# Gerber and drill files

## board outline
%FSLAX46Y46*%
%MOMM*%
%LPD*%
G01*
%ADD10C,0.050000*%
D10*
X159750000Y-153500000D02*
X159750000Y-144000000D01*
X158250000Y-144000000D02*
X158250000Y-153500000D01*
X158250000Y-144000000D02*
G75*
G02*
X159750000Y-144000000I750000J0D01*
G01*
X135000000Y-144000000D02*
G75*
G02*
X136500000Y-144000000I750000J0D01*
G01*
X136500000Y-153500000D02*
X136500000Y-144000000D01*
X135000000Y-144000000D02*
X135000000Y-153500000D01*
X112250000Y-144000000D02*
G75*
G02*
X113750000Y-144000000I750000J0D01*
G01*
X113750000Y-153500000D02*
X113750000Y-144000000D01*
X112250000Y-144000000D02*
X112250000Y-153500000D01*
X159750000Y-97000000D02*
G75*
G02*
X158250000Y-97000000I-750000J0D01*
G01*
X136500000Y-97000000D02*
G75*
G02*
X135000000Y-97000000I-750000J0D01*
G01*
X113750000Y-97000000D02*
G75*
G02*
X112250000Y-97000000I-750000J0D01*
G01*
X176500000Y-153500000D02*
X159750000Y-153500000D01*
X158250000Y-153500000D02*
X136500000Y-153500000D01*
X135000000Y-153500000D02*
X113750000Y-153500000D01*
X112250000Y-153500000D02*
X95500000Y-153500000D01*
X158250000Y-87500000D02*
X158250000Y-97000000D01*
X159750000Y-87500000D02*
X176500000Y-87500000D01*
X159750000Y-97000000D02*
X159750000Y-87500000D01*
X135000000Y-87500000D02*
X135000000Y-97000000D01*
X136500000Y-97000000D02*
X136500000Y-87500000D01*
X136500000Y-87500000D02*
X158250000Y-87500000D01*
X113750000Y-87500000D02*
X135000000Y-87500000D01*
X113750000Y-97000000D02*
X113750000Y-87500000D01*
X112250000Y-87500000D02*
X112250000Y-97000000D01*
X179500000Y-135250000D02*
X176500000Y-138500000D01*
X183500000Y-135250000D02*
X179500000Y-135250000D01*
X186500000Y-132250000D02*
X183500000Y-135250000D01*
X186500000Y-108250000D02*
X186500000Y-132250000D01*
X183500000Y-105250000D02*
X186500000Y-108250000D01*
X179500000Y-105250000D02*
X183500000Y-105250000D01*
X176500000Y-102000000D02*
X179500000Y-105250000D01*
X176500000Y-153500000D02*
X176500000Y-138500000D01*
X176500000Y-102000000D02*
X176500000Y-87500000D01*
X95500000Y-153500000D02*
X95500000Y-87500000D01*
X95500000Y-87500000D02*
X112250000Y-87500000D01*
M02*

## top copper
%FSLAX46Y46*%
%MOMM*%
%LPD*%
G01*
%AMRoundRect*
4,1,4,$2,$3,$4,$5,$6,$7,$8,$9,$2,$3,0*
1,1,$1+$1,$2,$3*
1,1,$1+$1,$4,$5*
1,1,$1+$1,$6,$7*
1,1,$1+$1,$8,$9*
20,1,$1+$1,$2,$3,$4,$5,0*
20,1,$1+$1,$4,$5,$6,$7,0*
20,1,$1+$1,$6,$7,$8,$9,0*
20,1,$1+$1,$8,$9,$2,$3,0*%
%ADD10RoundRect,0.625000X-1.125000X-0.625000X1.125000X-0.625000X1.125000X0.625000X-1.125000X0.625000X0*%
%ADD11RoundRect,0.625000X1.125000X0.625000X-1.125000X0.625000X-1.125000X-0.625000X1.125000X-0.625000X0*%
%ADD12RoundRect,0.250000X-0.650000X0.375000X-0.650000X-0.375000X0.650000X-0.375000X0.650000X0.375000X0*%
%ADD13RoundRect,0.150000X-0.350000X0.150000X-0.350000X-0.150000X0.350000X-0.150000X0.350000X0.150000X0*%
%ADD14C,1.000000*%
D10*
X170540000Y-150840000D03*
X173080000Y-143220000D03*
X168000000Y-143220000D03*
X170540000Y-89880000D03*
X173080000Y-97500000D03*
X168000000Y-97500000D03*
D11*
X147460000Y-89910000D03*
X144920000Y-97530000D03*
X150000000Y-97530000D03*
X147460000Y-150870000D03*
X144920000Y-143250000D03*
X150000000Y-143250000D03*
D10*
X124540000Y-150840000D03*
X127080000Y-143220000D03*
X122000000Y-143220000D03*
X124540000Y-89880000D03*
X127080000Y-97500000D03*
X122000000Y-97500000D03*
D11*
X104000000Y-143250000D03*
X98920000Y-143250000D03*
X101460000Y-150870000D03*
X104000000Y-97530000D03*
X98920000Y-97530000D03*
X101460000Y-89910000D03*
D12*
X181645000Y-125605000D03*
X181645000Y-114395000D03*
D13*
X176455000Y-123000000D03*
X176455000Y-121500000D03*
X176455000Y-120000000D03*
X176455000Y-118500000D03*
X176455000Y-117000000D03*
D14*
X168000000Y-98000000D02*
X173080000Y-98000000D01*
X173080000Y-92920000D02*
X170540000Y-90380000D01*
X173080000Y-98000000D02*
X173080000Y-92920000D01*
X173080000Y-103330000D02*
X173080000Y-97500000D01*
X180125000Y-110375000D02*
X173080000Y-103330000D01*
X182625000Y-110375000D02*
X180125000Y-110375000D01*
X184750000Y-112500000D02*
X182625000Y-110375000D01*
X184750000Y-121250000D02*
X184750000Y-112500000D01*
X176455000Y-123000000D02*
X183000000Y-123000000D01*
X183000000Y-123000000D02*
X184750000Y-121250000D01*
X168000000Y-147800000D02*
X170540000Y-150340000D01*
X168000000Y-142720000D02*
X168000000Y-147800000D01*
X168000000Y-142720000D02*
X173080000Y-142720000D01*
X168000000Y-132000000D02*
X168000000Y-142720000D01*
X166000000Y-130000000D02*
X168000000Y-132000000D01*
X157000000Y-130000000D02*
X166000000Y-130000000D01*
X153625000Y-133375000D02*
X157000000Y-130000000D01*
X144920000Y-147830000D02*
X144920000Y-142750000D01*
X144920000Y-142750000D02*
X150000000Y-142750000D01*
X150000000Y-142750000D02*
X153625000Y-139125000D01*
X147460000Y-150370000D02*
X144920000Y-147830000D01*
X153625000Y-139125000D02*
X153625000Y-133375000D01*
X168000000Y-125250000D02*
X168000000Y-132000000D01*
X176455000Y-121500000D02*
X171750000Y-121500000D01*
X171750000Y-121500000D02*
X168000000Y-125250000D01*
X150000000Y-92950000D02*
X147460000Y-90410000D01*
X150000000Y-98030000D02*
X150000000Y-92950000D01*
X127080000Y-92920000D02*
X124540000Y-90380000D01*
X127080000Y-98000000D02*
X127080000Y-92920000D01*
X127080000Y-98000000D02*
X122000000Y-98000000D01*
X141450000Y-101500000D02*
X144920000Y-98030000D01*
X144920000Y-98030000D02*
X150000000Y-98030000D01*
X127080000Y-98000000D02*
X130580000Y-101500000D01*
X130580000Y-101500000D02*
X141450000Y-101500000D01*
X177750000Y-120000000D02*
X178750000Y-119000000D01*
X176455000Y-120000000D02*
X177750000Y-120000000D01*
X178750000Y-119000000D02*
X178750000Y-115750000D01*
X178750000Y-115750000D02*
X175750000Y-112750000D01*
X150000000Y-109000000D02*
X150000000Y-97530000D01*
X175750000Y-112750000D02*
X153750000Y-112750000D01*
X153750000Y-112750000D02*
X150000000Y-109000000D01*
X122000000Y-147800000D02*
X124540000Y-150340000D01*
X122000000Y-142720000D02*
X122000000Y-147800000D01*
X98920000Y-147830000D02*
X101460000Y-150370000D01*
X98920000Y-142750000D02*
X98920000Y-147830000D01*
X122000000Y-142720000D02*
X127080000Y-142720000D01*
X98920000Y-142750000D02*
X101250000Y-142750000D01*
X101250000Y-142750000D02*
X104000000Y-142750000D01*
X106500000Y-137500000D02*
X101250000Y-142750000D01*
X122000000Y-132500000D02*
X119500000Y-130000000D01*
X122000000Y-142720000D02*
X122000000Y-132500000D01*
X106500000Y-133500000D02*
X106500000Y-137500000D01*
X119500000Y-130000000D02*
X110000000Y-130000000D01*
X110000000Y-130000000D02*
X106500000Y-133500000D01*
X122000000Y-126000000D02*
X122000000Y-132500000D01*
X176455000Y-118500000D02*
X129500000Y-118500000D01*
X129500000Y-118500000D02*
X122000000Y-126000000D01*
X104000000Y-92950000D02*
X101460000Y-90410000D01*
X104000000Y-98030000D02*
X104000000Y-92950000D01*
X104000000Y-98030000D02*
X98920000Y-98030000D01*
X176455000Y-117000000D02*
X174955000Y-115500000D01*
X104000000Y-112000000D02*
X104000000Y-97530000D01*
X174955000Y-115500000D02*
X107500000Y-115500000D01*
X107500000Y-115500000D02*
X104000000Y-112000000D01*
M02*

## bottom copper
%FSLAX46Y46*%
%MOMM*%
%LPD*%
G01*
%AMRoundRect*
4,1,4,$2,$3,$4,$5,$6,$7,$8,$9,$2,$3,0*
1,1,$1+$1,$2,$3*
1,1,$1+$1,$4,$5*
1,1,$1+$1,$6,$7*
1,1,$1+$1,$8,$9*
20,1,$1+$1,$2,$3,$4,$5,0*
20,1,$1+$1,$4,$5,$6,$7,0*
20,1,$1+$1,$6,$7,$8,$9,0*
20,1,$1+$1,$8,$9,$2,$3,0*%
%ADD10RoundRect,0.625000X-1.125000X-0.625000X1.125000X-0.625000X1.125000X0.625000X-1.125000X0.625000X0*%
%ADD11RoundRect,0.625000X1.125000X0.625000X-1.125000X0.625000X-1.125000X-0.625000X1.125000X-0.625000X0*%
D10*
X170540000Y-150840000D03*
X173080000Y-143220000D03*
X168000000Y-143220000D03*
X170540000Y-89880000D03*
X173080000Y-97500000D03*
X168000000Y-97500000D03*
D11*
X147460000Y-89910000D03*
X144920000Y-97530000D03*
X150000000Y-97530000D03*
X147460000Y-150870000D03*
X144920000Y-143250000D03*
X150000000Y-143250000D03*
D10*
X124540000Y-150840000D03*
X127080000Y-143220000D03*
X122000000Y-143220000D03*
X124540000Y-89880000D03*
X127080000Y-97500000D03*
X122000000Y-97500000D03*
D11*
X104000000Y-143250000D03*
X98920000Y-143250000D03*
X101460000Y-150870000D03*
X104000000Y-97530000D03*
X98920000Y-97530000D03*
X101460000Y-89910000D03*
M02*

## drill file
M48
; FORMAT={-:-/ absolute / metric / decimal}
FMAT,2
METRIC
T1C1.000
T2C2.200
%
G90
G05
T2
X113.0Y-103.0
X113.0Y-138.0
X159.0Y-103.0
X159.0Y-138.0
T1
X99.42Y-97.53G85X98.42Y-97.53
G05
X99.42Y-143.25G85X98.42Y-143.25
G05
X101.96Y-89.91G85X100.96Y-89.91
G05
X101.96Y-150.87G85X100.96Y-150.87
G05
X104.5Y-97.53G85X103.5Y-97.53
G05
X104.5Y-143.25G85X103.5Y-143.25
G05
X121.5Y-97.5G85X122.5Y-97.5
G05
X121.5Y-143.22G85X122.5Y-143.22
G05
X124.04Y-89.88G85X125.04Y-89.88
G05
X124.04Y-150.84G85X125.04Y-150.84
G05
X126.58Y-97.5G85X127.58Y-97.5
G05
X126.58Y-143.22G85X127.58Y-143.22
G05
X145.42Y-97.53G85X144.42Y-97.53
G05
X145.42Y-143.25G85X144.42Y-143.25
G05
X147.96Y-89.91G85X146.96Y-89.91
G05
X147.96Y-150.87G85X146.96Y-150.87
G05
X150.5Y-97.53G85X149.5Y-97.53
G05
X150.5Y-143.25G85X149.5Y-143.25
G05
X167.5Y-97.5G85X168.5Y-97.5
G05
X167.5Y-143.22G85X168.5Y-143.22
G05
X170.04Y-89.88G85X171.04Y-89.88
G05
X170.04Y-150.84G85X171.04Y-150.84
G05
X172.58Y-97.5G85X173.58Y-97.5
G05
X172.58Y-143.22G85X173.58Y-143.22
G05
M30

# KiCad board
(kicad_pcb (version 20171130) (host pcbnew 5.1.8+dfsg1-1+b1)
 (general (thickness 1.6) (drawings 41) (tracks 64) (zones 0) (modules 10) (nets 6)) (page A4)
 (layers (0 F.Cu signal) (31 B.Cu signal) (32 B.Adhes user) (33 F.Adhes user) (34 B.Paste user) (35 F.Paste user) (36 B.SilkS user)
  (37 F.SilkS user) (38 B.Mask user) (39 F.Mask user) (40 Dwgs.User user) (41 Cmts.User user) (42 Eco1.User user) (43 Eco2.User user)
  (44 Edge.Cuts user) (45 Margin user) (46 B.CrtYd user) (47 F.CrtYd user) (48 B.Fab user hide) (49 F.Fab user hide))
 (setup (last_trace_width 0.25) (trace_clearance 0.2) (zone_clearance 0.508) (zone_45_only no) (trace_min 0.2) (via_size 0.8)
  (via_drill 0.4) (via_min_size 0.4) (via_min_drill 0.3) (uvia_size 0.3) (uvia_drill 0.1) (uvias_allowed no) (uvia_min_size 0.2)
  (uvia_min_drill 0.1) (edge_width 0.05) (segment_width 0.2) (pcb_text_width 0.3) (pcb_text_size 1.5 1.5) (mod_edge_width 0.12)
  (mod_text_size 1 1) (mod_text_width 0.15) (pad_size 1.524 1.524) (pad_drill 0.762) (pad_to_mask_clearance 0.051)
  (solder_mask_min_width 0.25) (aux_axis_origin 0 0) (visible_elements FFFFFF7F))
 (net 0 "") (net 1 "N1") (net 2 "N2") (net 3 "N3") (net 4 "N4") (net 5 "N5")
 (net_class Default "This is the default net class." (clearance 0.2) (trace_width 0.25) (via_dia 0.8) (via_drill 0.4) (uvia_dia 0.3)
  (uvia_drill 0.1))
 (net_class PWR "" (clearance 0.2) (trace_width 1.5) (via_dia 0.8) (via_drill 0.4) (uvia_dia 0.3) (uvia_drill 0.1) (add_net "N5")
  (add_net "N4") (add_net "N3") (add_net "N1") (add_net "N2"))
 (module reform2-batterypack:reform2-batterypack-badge (layer F.Cu) (at 136 120.5 90)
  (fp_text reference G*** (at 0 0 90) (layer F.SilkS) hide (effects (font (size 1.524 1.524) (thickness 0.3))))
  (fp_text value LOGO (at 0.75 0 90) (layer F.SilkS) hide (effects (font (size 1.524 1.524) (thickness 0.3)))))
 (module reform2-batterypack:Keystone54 (layer F.Cu) (at 168 98)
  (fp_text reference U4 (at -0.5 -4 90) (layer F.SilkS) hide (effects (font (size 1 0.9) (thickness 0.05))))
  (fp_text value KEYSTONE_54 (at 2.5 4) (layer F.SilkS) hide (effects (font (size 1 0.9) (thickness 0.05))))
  (pad 6 thru_hole roundrect (at 2.54 52.84) (size 3.5 2.5) (drill oval 2 1) (layers *.Cu *.Mask) (roundrect_rratio 0.25) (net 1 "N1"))
  (pad 5 thru_hole roundrect (at 5.08 45.22) (size 3.5 2.5) (drill oval 2 1) (layers *.Cu *.Mask) (roundrect_rratio 0.25) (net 1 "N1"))
  (pad 4 thru_hole roundrect (at 0 45.22) (size 3.5 2.5) (drill oval 2 1) (layers *.Cu *.Mask) (roundrect_rratio 0.25) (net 1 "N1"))
  (pad 3 thru_hole roundrect (at 2.54 -8.12) (size 3.5 2.5) (drill oval 2 1) (layers *.Cu *.Mask) (roundrect_rratio 0.25) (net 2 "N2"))
  (pad 2 thru_hole roundrect (at 5.08 -0.5) (size 3.5 2.5) (drill oval 2 1) (layers *.Cu *.Mask) (roundrect_rratio 0.25) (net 2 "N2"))
  (pad 1 thru_hole roundrect (at 0 -0.5) (size 3.5 2.5) (drill oval 2 1) (layers *.Cu *.Mask) (roundrect_rratio 0.25) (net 2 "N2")))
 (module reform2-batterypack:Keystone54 (layer F.Cu) (at 150 142.75 180)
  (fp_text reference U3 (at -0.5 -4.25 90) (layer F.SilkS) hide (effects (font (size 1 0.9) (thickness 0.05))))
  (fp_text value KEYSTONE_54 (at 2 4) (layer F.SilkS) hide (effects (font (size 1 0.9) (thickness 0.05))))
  (pad 6 thru_hole roundrect (at 2.54 52.84 180) (size 3.5 2.5) (drill oval 2 1) (layers *.Cu *.Mask) (roundrect_rratio 0.25) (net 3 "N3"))
  (pad 5 thru_hole roundrect (at 5.08 45.22 180) (size 3.5 2.5) (drill oval 2 1) (layers *.Cu *.Mask) (roundrect_rratio 0.25) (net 3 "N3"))
  (pad 4 thru_hole roundrect (at 0 45.22 180) (size 3.5 2.5) (drill oval 2 1) (layers *.Cu *.Mask) (roundrect_rratio 0.25) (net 3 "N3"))
  (pad 3 thru_hole roundrect (at 2.54 -8.12 180) (size 3.5 2.5) (drill oval 2 1) (layers *.Cu *.Mask) (roundrect_rratio 0.25) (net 1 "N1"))
  (pad 2 thru_hole roundrect (at 5.08 -0.5 180) (size 3.5 2.5) (drill oval 2 1) (layers *.Cu *.Mask) (roundrect_rratio 0.25) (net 1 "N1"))
  (pad 1 thru_hole roundrect (at 0 -0.5 180) (size 3.5 2.5) (drill oval 2 1) (layers *.Cu *.Mask) (roundrect_rratio 0.25) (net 1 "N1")))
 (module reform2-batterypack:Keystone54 (layer F.Cu) (at 122 98)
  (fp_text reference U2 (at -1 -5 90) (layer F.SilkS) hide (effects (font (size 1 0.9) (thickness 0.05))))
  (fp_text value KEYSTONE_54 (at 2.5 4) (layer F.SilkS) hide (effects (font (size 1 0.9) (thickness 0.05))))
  (pad 6 thru_hole roundrect (at 2.54 52.84) (size 3.5 2.5) (drill oval 2 1) (layers *.Cu *.Mask) (roundrect_rratio 0.25) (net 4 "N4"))
  (pad 5 thru_hole roundrect (at 5.08 45.22) (size 3.5 2.5) (drill oval 2 1) (layers *.Cu *.Mask) (roundrect_rratio 0.25) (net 4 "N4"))
  (pad 4 thru_hole roundrect (at 0 45.22) (size 3.5 2.5) (drill oval 2 1) (layers *.Cu *.Mask) (roundrect_rratio 0.25) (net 4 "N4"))
  (pad 3 thru_hole roundrect (at 2.54 -8.12) (size 3.5 2.5) (drill oval 2 1) (layers *.Cu *.Mask) (roundrect_rratio 0.25) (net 3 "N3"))
  (pad 2 thru_hole roundrect (at 5.08 -0.5) (size 3.5 2.5) (drill oval 2 1) (layers *.Cu *.Mask) (roundrect_rratio 0.25) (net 3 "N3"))
  (pad 1 thru_hole roundrect (at 0 -0.5) (size 3.5 2.5) (drill oval 2 1) (layers *.Cu *.Mask) (roundrect_rratio 0.25) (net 3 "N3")))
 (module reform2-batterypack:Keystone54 (layer F.Cu) (at 104 142.75 180)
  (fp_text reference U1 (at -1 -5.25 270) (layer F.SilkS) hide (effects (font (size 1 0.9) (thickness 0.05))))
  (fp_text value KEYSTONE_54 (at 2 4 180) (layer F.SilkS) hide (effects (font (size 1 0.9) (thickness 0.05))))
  (pad 1 thru_hole roundrect (at 0 -0.5 180) (size 3.5 2.5) (drill oval 2 1) (layers *.Cu *.Mask) (roundrect_rratio 0.25) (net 4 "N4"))
  (pad 2 thru_hole roundrect (at 5.08 -0.5 180) (size 3.5 2.5) (drill oval 2 1) (layers *.Cu *.Mask) (roundrect_rratio 0.25) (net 4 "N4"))
  (pad 3 thru_hole roundrect (at 2.54 -8.12 180) (size 3.5 2.5) (drill oval 2 1) (layers *.Cu *.Mask) (roundrect_rratio 0.25) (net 4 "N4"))
  (pad 4 thru_hole roundrect (at 0 45.22 180) (size 3.5 2.5) (drill oval 2 1) (layers *.Cu *.Mask) (roundrect_rratio 0.25) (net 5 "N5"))
  (pad 5 thru_hole roundrect (at 5.08 45.22 180) (size 3.5 2.5) (drill oval 2 1) (layers *.Cu *.Mask) (roundrect_rratio 0.25) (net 5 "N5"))
  (pad 6 thru_hole roundrect (at 2.54 52.84 180) (size 3.5 2.5) (drill oval 2 1) (layers *.Cu *.Mask) (roundrect_rratio 0.25) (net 5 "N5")))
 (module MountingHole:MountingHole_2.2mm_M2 (layer F.Cu) (at 159 138)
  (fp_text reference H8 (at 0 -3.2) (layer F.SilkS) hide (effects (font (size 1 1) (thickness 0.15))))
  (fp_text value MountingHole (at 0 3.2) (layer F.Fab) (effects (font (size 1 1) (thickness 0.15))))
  (pad 1 np_thru_hole circle (at 0 0) (size 2.2 2.2) (drill 2.2) (layers *.Cu *.Mask)))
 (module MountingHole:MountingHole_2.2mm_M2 (layer F.Cu) (at 113 138)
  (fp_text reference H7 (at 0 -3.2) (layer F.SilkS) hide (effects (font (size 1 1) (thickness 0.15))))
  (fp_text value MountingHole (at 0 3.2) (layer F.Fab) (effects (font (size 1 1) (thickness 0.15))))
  (pad 1 np_thru_hole circle (at 0 0) (size 2.2 2.2) (drill 2.2) (layers *.Cu *.Mask)))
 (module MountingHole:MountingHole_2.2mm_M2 (layer F.Cu) (at 159 103)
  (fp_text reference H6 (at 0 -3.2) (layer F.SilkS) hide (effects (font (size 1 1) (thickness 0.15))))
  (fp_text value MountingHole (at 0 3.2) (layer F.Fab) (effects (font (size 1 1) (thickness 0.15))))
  (pad 1 np_thru_hole circle (at 0 0) (size 2.2 2.2) (drill 2.2) (layers *.Cu *.Mask)))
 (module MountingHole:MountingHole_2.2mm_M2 (layer F.Cu) (at 113 103)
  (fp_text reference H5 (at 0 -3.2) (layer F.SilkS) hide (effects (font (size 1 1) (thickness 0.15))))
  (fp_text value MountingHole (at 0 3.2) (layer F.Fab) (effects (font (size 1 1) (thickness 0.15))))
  (pad 1 np_thru_hole circle (at 0 0) (size 2.2 2.2) (drill 2.2) (layers *.Cu *.Mask)))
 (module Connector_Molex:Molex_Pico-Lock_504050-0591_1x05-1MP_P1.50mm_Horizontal (layer F.Cu) (at 179.25 120 270)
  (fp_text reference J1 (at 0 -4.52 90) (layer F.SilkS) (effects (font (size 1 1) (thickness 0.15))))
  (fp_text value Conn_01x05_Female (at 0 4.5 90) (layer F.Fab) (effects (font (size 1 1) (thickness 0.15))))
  (pad MP smd roundrect (at 5.605 -2.395 270) (size 1.25 1.8) (layers F.Cu F.Paste F.Mask) (roundrect_rratio 0.2))
  (pad MP smd roundrect (at -5.605 -2.395 270) (size 1.25 1.8) (layers F.Cu F.Paste F.Mask) (roundrect_rratio 0.2))
  (pad 5 smd roundrect (at 3 2.795 270) (size 0.6 1) (layers F.Cu F.Paste F.Mask) (roundrect_rratio 0.25) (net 2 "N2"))
  (pad 4 smd roundrect (at 1.5 2.795 270) (size 0.6 1) (layers F.Cu F.Paste F.Mask) (roundrect_rratio 0.25) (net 1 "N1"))
  (pad 3 smd roundrect (at 0 2.795 270) (size 0.6 1) (layers F.Cu F.Paste F.Mask) (roundrect_rratio 0.25) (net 3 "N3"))
  (pad 2 smd roundrect (at -1.5 2.795 270) (size 0.6 1) (layers F.Cu F.Paste F.Mask) (roundrect_rratio 0.25) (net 4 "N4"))
  (pad 1 smd roundrect (at -3 2.795 270) (size 0.6 1) (layers F.Cu F.Paste F.Mask) (roundrect_rratio 0.25) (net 5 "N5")))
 (gr_line (start 159.75 153.5) (end 159.75 144) (layer Edge.Cuts) (width 0.05))
 (gr_line (start 158.25 144) (end 158.25 153.5) (layer Edge.Cuts) (width 0.05))
 (gr_arc (start 159 144) (end 159.75 144) (angle -180) (layer Edge.Cuts) (width 0.05))
 (gr_arc (start 135.75 144) (end 136.5 144) (angle -180) (layer Edge.Cuts) (width 0.05))
 (gr_line (start 136.5 153.5) (end 136.5 144) (layer Edge.Cuts) (width 0.05))
 (gr_line (start 135 144) (end 135 153.5) (layer Edge.Cuts) (width 0.05))
 (gr_arc (start 113 144) (end 113.75 144) (angle -180) (layer Edge.Cuts) (width 0.05))
 (gr_line (start 113.75 153.5) (end 113.75 144) (layer Edge.Cuts) (width 0.05))
 (gr_line (start 112.25 144) (end 112.25 153.5) (layer Edge.Cuts) (width 0.05))
 (gr_arc (start 159 97) (end 158.25 97) (angle -180) (layer Edge.Cuts) (width 0.05))
 (gr_arc (start 135.75 97) (end 135 97) (angle -180) (layer Edge.Cuts) (width 0.05))
 (gr_arc (start 113 97) (end 112.25 97) (angle -180) (layer Edge.Cuts) (width 0.05))
 (gr_line (start 176.5 153.5) (end 159.75 153.5) (layer Edge.Cuts) (width 0.05))
 (gr_line (start 158.25 153.5) (end 136.5 153.5) (layer Edge.Cuts) (width 0.05))
 (gr_line (start 135 153.5) (end 113.75 153.5) (layer Edge.Cuts) (width 0.05))
 (gr_line (start 112.25 153.5) (end 95.5 153.5) (layer Edge.Cuts) (width 0.05))
 (gr_line (start 158.25 87.5) (end 158.25 97) (layer Edge.Cuts) (width 0.05))
 (gr_line (start 159.75 87.5) (end 176.5 87.5) (layer Edge.Cuts) (width 0.05))
 (gr_line (start 159.75 97) (end 159.75 87.5) (layer Edge.Cuts) (width 0.05))
 (gr_line (start 135 87.5) (end 135 97) (layer Edge.Cuts) (width 0.05))
 (gr_line (start 136.5 97) (end 136.5 87.5) (layer Edge.Cuts) (width 0.05))
 (gr_line (start 136.5 87.5) (end 158.25 87.5) (layer Edge.Cuts) (width 0.05))
 (gr_line (start 113.75 87.5) (end 135 87.5) (layer Edge.Cuts) (width 0.05))
 (gr_line (start 113.75 97) (end 113.75 87.5) (layer Edge.Cuts) (width 0.05))
 (gr_line (start 112.25 87.5) (end 112.25 97) (layer Edge.Cuts) (width 0.05))
 (gr_line (start 179.5 135.25) (end 176.5 138.5) (layer Edge.Cuts) (width 0.05))
 (gr_line (start 183.5 135.25) (end 179.5 135.25) (layer Edge.Cuts) (width 0.05))
 (gr_line (start 186.5 132.25) (end 183.5 135.25) (layer Edge.Cuts) (width 0.05))
 (gr_line (start 186.5 108.25) (end 186.5 132.25) (layer Edge.Cuts) (width 0.05))
 (gr_line (start 183.5 105.25) (end 186.5 108.25) (layer Edge.Cuts) (width 0.05))
 (gr_line (start 179.5 105.25) (end 183.5 105.25) (layer Edge.Cuts) (width 0.05))
 (gr_line (start 176.5 102) (end 179.5 105.25) (layer Edge.Cuts) (width 0.05))
 (gr_line (start 176.5 153.5) (end 176.5 138.5) (layer Edge.Cuts) (width 0.05))
 (gr_line (start 176.5 102) (end 176.5 87.5) (layer Edge.Cuts) (width 0.05))
 (gr_line (start 95.5 153.5) (end 95.5 87.5) (layer Edge.Cuts) (width 0.05))
 (gr_line (start 95.5 87.5) (end 112.25 87.5) (layer Edge.Cuts) (width 0.05))
 (segment (start 168 98) (end 173.08 98) (width 1) (layer F.Cu) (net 2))
 (segment (start 173.08 92.92) (end 170.54 90.38) (width 1) (layer F.Cu) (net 2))
 (segment (start 173.08 98) (end 173.08 92.92) (width 1) (layer F.Cu) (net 2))
 (segment (start 173.08 103.33) (end 173.08 97.5) (width 1) (layer F.Cu) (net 2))
 (segment (start 180.125 110.375) (end 173.08 103.33) (width 1) (layer F.Cu) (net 2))
 (segment (start 182.625 110.375) (end 180.125 110.375) (width 1) (layer F.Cu) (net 2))
 (segment (start 184.75 112.5) (end 182.625 110.375) (width 1) (layer F.Cu) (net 2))
 (segment (start 184.75 121.25) (end 184.75 112.5) (width 1) (layer F.Cu) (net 2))
 (segment (start 176.455 123) (end 183 123) (width 1) (layer F.Cu) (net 2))
 (segment (start 183 123) (end 184.75 121.25) (width 1) (layer F.Cu) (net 2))
 (segment (start 168 147.8) (end 170.54 150.34) (width 1) (layer F.Cu) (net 1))
 (segment (start 168 142.72) (end 168 147.8) (width 1) (layer F.Cu) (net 1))
 (segment (start 168 142.72) (end 173.08 142.72) (width 1) (layer F.Cu) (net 1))
 (segment (start 168 132) (end 168 142.72) (width 1) (layer F.Cu) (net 1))
 (segment (start 166 130) (end 168 132) (width 1) (layer F.Cu) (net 1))
 (segment (start 157 130) (end 166 130) (width 1) (layer F.Cu) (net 1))
 (segment (start 153.625 133.375) (end 157 130) (width 1) (layer F.Cu) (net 1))
 (segment (start 144.92 147.83) (end 144.92 142.75) (width 1) (layer F.Cu) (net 1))
 (segment (start 144.92 142.75) (end 150 142.75) (width 1) (layer F.Cu) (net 1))
 (segment (start 150 142.75) (end 153.625 139.125) (width 1) (layer F.Cu) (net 1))
 (segment (start 147.46 150.37) (end 144.92 147.83) (width 1) (layer F.Cu) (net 1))
 (segment (start 153.625 139.125) (end 153.625 133.375) (width 1) (layer F.Cu) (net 1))
 (segment (start 168 125.25) (end 168 132) (width 1) (layer F.Cu) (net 1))
 (segment (start 176.455 121.5) (end 171.75 121.5) (width 1) (layer F.Cu) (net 1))
 (segment (start 171.75 121.5) (end 168 125.25) (width 1) (layer F.Cu) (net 1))
 (segment (start 150 92.95) (end 147.46 90.41) (width 1) (layer F.Cu) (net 3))
 (segment (start 150 98.03) (end 150 92.95) (width 1) (layer F.Cu) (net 3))
 (segment (start 127.08 92.92) (end 124.54 90.38) (width 1) (layer F.Cu) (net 3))
 (segment (start 127.08 98) (end 127.08 92.92) (width 1) (layer F.Cu) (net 3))
 (segment (start 127.08 98) (end 122 98) (width 1) (layer F.Cu) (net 3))
 (segment (start 141.45 101.5) (end 144.92 98.03) (width 1) (layer F.Cu) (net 3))
 (segment (start 144.92 98.03) (end 150 98.03) (width 1) (layer F.Cu) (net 3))
 (segment (start 127.08 98) (end 130.58 101.5) (width 1) (layer F.Cu) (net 3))
 (segment (start 130.58 101.5) (end 141.45 101.5) (width 1) (layer F.Cu) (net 3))
 (segment (start 177.75 120) (end 178.75 119) (width 1) (layer F.Cu) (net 3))
 (segment (start 176.455 120) (end 177.75 120) (width 1) (layer F.Cu) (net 3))
 (segment (start 178.75 119) (end 178.75 115.75) (width 1) (layer F.Cu) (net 3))
 (segment (start 178.75 115.75) (end 175.75 112.75) (width 1) (layer F.Cu) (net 3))
 (segment (start 150 109) (end 150 97.53) (width 1) (layer F.Cu) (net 3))
 (segment (start 175.75 112.75) (end 153.75 112.75) (width 1) (layer F.Cu) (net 3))
 (segment (start 153.75 112.75) (end 150 109) (width 1) (layer F.Cu) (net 3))
 (segment (start 122 147.8) (end 124.54 150.34) (width 1) (layer F.Cu) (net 4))
 (segment (start 122 142.72) (end 122 147.8) (width 1) (layer F.Cu) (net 4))
 (segment (start 98.92 147.83) (end 101.46 150.37) (width 1) (layer F.Cu) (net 4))
 (segment (start 98.92 142.75) (end 98.92 147.83) (width 1) (layer F.Cu) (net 4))
 (segment (start 122 142.72) (end 127.08 142.72) (width 1) (layer F.Cu) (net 4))
 (segment (start 98.92 142.75) (end 101.25 142.75) (width 1) (layer F.Cu) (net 4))
 (segment (start 101.25 142.75) (end 104 142.75) (width 1) (layer F.Cu) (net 4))
 (segment (start 106.5 137.5) (end 101.25 142.75) (width 1) (layer F.Cu) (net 4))
 (segment (start 122 132.5) (end 119.5 130) (width 1) (layer F.Cu) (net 4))
 (segment (start 122 142.72) (end 122 132.5) (width 1) (layer F.Cu) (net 4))
 (segment (start 106.5 133.5) (end 106.5 137.5) (width 1) (layer F.Cu) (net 4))
 (segment (start 119.5 130) (end 110 130) (width 1) (layer F.Cu) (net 4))
 (segment (start 110 130) (end 106.5 133.5) (width 1) (layer F.Cu) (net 4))
 (segment (start 122 126) (end 122 132.5) (width 1) (layer F.Cu) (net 4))
 (segment (start 176.455 118.5) (end 129.5 118.5) (width 1) (layer F.Cu) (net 4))
 (segment (start 129.5 118.5) (end 122 126) (width 1) (layer F.Cu) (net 4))
 (segment (start 104 92.95) (end 101.46 90.41) (width 1) (layer F.Cu) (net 5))
 (segment (start 104 98.03) (end 104 92.95) (width 1) (layer F.Cu) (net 5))
 (segment (start 104 98.03) (end 98.92 98.03) (width 1) (layer F.Cu) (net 5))
 (segment (start 176.455 117) (end 174.955 115.5) (width 1) (layer F.Cu) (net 5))
 (segment (start 104 112) (end 104 97.53) (width 1) (layer F.Cu) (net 5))
 (segment (start 174.955 115.5) (end 107.5 115.5) (width 1) (layer F.Cu) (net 5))
 (segment (start 107.5 115.5) (end 104 112) (width 1) (layer F.Cu) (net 5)))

